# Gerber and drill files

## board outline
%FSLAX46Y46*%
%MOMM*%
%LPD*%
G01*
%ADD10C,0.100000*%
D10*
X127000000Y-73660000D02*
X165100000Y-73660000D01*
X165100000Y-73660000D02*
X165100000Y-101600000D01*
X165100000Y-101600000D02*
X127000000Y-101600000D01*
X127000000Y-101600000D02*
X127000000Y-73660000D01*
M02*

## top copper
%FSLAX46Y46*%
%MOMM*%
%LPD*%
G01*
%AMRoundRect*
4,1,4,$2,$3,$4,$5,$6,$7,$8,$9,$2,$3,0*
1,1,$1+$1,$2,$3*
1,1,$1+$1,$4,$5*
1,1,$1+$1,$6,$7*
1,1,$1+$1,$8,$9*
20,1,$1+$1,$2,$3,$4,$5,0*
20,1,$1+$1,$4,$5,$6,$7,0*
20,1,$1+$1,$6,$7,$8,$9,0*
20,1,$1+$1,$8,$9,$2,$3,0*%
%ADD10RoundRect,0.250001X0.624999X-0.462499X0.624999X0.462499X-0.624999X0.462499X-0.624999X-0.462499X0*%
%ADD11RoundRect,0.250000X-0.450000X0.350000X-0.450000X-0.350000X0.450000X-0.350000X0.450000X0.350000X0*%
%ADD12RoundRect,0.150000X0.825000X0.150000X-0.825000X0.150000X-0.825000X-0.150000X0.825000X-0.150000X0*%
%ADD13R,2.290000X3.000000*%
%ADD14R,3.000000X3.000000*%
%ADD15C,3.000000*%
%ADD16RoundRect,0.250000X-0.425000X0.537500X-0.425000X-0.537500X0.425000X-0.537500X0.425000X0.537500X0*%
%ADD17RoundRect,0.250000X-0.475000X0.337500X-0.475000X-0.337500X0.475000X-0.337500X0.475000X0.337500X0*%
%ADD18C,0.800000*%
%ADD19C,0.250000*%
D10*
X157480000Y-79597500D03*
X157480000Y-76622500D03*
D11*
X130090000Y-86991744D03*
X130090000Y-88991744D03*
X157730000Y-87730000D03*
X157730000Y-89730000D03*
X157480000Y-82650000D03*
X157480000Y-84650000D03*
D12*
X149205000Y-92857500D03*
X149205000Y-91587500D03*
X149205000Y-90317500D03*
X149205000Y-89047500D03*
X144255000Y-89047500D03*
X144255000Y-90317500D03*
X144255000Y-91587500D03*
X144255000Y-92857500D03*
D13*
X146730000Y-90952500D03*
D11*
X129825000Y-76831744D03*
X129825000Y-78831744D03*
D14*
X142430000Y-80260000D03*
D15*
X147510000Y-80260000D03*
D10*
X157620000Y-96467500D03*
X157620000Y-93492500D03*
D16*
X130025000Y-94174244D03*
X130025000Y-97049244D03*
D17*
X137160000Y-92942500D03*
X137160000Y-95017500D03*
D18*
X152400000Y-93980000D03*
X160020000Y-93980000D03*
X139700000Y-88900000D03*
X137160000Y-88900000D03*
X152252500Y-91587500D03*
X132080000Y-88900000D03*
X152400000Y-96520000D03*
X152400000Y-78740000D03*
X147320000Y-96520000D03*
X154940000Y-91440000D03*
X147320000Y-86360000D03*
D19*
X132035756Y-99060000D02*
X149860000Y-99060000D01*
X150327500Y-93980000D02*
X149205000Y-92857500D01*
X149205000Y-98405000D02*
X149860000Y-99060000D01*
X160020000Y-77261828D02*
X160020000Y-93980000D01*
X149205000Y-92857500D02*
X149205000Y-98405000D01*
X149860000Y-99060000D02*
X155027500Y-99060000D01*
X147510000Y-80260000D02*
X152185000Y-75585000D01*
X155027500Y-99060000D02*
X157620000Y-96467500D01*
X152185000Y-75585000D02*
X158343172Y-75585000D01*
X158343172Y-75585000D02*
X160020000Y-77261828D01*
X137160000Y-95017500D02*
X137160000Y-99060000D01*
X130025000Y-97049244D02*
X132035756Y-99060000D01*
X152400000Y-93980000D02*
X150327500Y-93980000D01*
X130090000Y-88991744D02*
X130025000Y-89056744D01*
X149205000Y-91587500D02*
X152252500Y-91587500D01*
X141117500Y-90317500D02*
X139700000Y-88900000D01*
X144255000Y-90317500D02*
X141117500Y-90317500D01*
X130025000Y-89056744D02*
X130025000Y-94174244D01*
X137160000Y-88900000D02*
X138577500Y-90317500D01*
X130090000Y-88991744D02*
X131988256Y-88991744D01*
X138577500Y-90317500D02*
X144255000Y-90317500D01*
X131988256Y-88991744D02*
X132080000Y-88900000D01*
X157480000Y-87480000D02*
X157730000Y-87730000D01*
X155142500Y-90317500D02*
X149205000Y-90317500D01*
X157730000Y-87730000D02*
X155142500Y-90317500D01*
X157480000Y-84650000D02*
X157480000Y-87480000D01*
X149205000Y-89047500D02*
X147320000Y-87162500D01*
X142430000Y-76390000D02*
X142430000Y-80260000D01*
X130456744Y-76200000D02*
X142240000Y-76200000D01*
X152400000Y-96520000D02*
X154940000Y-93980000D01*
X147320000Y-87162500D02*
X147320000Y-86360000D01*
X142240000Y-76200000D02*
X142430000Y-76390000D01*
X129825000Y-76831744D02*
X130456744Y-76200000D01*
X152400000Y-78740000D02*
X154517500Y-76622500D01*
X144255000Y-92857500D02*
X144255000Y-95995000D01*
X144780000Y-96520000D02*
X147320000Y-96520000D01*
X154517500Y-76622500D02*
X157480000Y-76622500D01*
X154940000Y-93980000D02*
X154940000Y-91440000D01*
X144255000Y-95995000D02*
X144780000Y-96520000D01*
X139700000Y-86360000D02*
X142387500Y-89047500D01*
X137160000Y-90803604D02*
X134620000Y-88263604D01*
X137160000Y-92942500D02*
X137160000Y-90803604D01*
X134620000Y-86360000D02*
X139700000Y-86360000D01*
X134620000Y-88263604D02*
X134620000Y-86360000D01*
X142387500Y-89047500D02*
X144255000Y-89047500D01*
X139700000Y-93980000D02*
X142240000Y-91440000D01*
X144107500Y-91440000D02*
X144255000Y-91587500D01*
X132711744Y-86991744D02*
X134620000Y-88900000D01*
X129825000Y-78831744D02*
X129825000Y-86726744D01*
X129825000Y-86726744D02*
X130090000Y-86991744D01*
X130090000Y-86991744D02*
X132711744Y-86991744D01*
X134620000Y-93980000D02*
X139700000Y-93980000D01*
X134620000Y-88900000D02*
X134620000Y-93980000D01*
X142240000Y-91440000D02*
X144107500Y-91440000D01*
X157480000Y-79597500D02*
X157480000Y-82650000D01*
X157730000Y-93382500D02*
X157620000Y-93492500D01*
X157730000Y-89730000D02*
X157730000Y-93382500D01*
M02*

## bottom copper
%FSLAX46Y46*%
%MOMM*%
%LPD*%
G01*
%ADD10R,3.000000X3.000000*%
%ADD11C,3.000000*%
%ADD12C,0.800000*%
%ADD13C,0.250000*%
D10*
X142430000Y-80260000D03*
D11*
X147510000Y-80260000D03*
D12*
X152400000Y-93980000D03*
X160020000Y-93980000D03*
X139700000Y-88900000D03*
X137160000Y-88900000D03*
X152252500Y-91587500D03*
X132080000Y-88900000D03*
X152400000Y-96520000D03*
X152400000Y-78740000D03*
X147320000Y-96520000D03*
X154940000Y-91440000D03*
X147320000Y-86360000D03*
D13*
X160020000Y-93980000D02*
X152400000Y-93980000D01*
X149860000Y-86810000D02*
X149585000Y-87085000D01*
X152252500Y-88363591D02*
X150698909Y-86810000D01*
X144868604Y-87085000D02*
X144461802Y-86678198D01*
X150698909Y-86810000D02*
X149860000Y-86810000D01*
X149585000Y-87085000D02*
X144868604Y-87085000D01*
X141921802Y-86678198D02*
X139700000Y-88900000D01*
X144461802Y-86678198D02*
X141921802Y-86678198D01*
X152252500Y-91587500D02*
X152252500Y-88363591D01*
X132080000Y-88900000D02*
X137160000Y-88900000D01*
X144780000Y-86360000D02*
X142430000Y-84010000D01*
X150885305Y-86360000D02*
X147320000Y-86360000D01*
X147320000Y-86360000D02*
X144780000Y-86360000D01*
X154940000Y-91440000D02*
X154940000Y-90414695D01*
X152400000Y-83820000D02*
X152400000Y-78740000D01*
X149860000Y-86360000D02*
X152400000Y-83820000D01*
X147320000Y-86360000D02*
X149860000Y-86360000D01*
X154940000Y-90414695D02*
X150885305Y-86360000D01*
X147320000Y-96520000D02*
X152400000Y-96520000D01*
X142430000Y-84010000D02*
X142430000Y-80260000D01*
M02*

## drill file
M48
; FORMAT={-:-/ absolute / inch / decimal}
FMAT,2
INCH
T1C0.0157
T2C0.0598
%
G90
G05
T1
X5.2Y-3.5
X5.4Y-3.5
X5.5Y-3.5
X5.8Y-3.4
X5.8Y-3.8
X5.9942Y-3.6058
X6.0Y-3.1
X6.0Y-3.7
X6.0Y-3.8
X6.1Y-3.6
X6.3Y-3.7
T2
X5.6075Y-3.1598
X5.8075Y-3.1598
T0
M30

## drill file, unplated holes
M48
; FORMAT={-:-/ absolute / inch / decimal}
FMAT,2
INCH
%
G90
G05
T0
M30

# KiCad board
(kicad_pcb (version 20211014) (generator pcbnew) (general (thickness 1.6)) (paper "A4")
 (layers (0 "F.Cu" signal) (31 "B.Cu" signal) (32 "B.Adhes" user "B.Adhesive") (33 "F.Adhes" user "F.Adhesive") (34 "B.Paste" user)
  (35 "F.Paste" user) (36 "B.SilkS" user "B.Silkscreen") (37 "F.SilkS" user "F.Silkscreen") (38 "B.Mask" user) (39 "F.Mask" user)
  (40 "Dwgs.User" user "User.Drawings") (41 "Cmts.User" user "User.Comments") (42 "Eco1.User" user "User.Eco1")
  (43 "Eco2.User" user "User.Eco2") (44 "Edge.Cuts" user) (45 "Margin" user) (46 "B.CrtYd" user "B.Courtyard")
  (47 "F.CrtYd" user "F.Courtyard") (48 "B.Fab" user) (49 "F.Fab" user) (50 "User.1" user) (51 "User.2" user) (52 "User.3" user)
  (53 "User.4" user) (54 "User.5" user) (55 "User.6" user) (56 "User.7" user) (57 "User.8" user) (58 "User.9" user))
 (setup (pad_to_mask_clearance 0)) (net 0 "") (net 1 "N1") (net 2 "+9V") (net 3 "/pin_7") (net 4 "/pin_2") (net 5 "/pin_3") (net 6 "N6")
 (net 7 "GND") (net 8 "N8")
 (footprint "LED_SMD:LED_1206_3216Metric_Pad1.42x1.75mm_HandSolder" (layer "F.Cu") (at 157.48 78.11 90)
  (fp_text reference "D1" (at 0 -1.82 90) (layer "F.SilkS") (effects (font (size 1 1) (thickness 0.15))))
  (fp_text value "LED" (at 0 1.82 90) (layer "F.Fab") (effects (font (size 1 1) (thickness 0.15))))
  (pad "1" smd roundrect (at -1.4875 0 90) (size 1.425 1.75) (layers "F.Cu" "F.Paste" "F.Mask") (roundrect_rratio 0.1754392982) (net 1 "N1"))
  (pad "2" smd roundrect (at 1.4875 0 90) (size 1.425 1.75) (layers "F.Cu" "F.Paste" "F.Mask") (roundrect_rratio 0.1754392982) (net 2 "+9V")))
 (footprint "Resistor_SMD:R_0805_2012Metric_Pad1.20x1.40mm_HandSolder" (layer "F.Cu") (at 130.09 87.991744 -90)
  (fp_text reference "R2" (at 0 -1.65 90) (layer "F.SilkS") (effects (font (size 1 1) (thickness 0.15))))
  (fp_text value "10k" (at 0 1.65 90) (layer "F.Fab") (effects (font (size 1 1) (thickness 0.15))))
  (pad "1" smd roundrect (at -1 0 270) (size 1.2 1.4) (layers "F.Cu" "F.Paste" "F.Mask") (roundrect_rratio 0.2083333333) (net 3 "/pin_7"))
  (pad "2" smd roundrect (at 1 0 270) (size 1.2 1.4) (layers "F.Cu" "F.Paste" "F.Mask") (roundrect_rratio 0.2083333333) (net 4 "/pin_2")))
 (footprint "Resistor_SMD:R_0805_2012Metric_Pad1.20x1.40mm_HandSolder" (layer "F.Cu") (at 157.73 88.73 -90)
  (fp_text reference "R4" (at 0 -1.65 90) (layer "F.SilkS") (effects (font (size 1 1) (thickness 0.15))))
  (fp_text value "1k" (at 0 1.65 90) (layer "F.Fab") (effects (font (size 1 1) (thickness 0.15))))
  (pad "1" smd roundrect (at -1 0 270) (size 1.2 1.4) (layers "F.Cu" "F.Paste" "F.Mask") (roundrect_rratio 0.2083333333) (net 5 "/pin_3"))
  (pad "2" smd roundrect (at 1 0 270) (size 1.2 1.4) (layers "F.Cu" "F.Paste" "F.Mask") (roundrect_rratio 0.2083333333) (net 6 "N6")))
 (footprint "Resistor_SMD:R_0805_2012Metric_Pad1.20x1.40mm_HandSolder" (layer "F.Cu") (at 157.48 83.65 -90)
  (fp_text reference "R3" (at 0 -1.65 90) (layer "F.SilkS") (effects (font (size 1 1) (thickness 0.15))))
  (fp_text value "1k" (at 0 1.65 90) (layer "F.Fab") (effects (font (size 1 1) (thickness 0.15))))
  (pad "1" smd roundrect (at -1 0 270) (size 1.2 1.4) (layers "F.Cu" "F.Paste" "F.Mask") (roundrect_rratio 0.2083333333) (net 1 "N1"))
  (pad "2" smd roundrect (at 1 0 270) (size 1.2 1.4) (layers "F.Cu" "F.Paste" "F.Mask") (roundrect_rratio 0.2083333333) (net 5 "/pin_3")))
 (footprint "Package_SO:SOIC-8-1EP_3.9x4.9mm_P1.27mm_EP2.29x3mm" (layer "F.Cu") (at 146.73 90.9525 180)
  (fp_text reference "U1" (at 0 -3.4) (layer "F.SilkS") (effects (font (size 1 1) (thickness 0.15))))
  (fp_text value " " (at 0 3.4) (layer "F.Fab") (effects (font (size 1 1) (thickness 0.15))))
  (pad "" smd roundrect (at -0.57 0.75 180) (size 0.92 1.21) (layers "F.Paste") (roundrect_rratio 0.25))
  (pad "" smd roundrect (at 0.57 -0.75 180) (size 0.92 1.21) (layers "F.Paste") (roundrect_rratio 0.25))
  (pad "" smd roundrect (at -0.57 -0.75 180) (size 0.92 1.21) (layers "F.Paste") (roundrect_rratio 0.25))
  (pad "" smd roundrect (at 0.57 0.75 180) (size 0.92 1.21) (layers "F.Paste") (roundrect_rratio 0.25))
  (pad "1" smd roundrect (at -2.475 -1.905 180) (size 1.95 0.6) (layers "F.Cu" "F.Paste" "F.Mask") (roundrect_rratio 0.25) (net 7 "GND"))
  (pad "2" smd roundrect (at -2.475 -0.635 180) (size 1.95 0.6) (layers "F.Cu" "F.Paste" "F.Mask") (roundrect_rratio 0.25) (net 4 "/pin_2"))
  (pad "3" smd roundrect (at -2.475 0.635 180) (size 1.95 0.6) (layers "F.Cu" "F.Paste" "F.Mask") (roundrect_rratio 0.25) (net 5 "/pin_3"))
  (pad "4" smd roundrect (at -2.475 1.905 180) (size 1.95 0.6) (layers "F.Cu" "F.Paste" "F.Mask") (roundrect_rratio 0.25) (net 2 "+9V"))
  (pad "5" smd roundrect (at 2.475 1.905 180) (size 1.95 0.6) (layers "F.Cu" "F.Paste" "F.Mask") (roundrect_rratio 0.25) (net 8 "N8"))
  (pad "6" smd roundrect (at 2.475 0.635 180) (size 1.95 0.6) (layers "F.Cu" "F.Paste" "F.Mask") (roundrect_rratio 0.25) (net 4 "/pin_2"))
  (pad "7" smd roundrect (at 2.475 -0.635 180) (size 1.95 0.6) (layers "F.Cu" "F.Paste" "F.Mask") (roundrect_rratio 0.25) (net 3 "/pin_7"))
  (pad "8" smd roundrect (at 2.475 -1.905 180) (size 1.95 0.6) (layers "F.Cu" "F.Paste" "F.Mask") (roundrect_rratio 0.25) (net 2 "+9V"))
  (pad "9" smd rect (at 0 0 180) (size 2.29 3) (layers "F.Cu" "F.Mask")))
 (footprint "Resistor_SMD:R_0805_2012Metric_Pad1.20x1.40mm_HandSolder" (layer "F.Cu") (at 129.825 77.831744 -90)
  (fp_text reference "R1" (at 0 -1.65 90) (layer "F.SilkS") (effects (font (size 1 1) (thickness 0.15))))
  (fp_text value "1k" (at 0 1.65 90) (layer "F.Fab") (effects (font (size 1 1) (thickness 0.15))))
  (pad "1" smd roundrect (at -1 0 270) (size 1.2 1.4) (layers "F.Cu" "F.Paste" "F.Mask") (roundrect_rratio 0.2083333333) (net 2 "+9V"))
  (pad "2" smd roundrect (at 1 0 270) (size 1.2 1.4) (layers "F.Cu" "F.Paste" "F.Mask") (roundrect_rratio 0.2083333333) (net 3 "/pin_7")))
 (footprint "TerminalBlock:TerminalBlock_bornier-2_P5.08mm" (layer "F.Cu") (at 142.43 80.26)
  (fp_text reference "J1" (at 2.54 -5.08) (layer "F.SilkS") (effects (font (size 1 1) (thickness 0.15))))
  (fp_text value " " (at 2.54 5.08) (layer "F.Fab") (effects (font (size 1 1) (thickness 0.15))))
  (pad "1" thru_hole rect (at 0 0) (size 3 3) (drill 1.52) (layers *.Cu *.Mask) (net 2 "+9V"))
  (pad "2" thru_hole circle (at 5.08 0) (size 3 3) (drill 1.52) (layers *.Cu *.Mask) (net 7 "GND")))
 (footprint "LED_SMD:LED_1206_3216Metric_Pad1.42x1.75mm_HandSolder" (layer "F.Cu") (at 157.62 94.98 90)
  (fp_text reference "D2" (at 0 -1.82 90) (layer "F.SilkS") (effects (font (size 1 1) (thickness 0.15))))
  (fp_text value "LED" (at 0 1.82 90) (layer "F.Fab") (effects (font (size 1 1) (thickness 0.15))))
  (pad "1" smd roundrect (at -1.4875 0 90) (size 1.425 1.75) (layers "F.Cu" "F.Paste" "F.Mask") (roundrect_rratio 0.1754392982)
   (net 7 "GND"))
  (pad "2" smd roundrect (at 1.4875 0 90) (size 1.425 1.75) (layers "F.Cu" "F.Paste" "F.Mask") (roundrect_rratio 0.1754392982) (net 6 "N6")))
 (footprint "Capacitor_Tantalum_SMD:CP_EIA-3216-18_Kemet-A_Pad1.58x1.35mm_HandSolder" (layer "F.Cu") (at 130.025 95.611744 -90)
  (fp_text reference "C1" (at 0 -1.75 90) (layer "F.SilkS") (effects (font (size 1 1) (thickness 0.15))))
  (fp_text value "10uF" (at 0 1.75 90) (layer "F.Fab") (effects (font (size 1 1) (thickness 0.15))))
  (pad "1" smd roundrect (at -1.4375 0 270) (size 1.575 1.35) (layers "F.Cu" "F.Paste" "F.Mask") (roundrect_rratio 0.1851851852)
   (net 4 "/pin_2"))
  (pad "2" smd roundrect (at 1.4375 0 270) (size 1.575 1.35) (layers "F.Cu" "F.Paste" "F.Mask") (roundrect_rratio 0.1851851852)
   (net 7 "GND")))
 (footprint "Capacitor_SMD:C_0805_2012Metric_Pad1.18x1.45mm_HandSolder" (layer "F.Cu") (at 137.16 93.98 -90)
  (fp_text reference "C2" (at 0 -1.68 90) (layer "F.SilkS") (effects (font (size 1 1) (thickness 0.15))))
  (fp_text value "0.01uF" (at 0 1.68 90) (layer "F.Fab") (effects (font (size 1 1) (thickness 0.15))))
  (pad "1" smd roundrect (at -1.0375 0 270) (size 1.175 1.45) (layers "F.Cu" "F.Paste" "F.Mask") (roundrect_rratio 0.2127659574)
   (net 8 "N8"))
  (pad "2" smd roundrect (at 1.0375 0 270) (size 1.175 1.45) (layers "F.Cu" "F.Paste" "F.Mask") (roundrect_rratio 0.2127659574)
   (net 7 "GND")))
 (gr_rect (start 127 73.66) (end 165.1 101.6) (layer "Edge.Cuts") (width 0.1) (fill none))
 (segment (start 132.035756 99.06) (end 149.86 99.06) (width 0.25) (layer "F.Cu") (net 7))
 (segment (start 150.3275 93.98) (end 149.205 92.8575) (width 0.25) (layer "F.Cu") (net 7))
 (segment (start 149.205 98.405) (end 149.86 99.06) (width 0.25) (layer "F.Cu") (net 7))
 (segment (start 160.02 77.261828) (end 160.02 93.98) (width 0.25) (layer "F.Cu") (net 7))
 (segment (start 149.205 92.8575) (end 149.205 98.405) (width 0.25) (layer "F.Cu") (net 7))
 (segment (start 149.86 99.06) (end 155.0275 99.06) (width 0.25) (layer "F.Cu") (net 7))
 (segment (start 147.51 80.26) (end 152.185 75.585) (width 0.25) (layer "F.Cu") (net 7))
 (segment (start 155.0275 99.06) (end 157.62 96.4675) (width 0.25) (layer "F.Cu") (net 7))
 (segment (start 152.185 75.585) (end 158.343172 75.585) (width 0.25) (layer "F.Cu") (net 7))
 (segment (start 158.343172 75.585) (end 160.02 77.261828) (width 0.25) (layer "F.Cu") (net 7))
 (segment (start 137.16 95.0175) (end 137.16 99.06) (width 0.25) (layer "F.Cu") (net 7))
 (segment (start 130.025 97.049244) (end 132.035756 99.06) (width 0.25) (layer "F.Cu") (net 7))
 (segment (start 152.4 93.98) (end 150.3275 93.98) (width 0.25) (layer "F.Cu") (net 7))
 (via (at 152.4 93.98) (size 0.8) (drill 0.4) (layers "F.Cu" "B.Cu") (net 7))
 (via (at 160.02 93.98) (size 0.8) (drill 0.4) (layers "F.Cu" "B.Cu") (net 7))
 (segment (start 160.02 93.98) (end 152.4 93.98) (width 0.25) (layer "B.Cu") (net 7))
 (segment (start 130.09 88.991744) (end 130.025 89.056744) (width 0.25) (layer "F.Cu") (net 4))
 (segment (start 149.205 91.5875) (end 152.2525 91.5875) (width 0.25) (layer "F.Cu") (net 4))
 (segment (start 141.1175 90.3175) (end 139.7 88.9) (width 0.25) (layer "F.Cu") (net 4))
 (segment (start 144.255 90.3175) (end 141.1175 90.3175) (width 0.25) (layer "F.Cu") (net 4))
 (segment (start 130.025 89.056744) (end 130.025 94.174244) (width 0.25) (layer "F.Cu") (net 4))
 (segment (start 137.16 88.9) (end 138.5775 90.3175) (width 0.25) (layer "F.Cu") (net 4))
 (segment (start 130.09 88.991744) (end 131.988256 88.991744) (width 0.25) (layer "F.Cu") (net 4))
 (segment (start 138.5775 90.3175) (end 144.255 90.3175) (width 0.25) (layer "F.Cu") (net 4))
 (segment (start 131.988256 88.991744) (end 132.08 88.9) (width 0.25) (layer "F.Cu") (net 4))
 (via (at 139.7 88.9) (size 0.8) (drill 0.4) (layers "F.Cu" "B.Cu") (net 4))
 (via (at 137.16 88.9) (size 0.8) (drill 0.4) (layers "F.Cu" "B.Cu") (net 4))
 (via (at 152.2525 91.5875) (size 0.8) (drill 0.4) (layers "F.Cu" "B.Cu") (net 4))
 (via (at 132.08 88.9) (size 0.8) (drill 0.4) (layers "F.Cu" "B.Cu") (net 4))
 (segment (start 149.86 86.81) (end 149.585 87.085) (width 0.25) (layer "B.Cu") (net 4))
 (segment (start 152.2525 88.363591) (end 150.698909 86.81) (width 0.25) (layer "B.Cu") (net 4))
 (segment (start 144.868604 87.085) (end 144.461802 86.678198) (width 0.25) (layer "B.Cu") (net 4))
 (segment (start 150.698909 86.81) (end 149.86 86.81) (width 0.25) (layer "B.Cu") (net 4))
 (segment (start 149.585 87.085) (end 144.868604 87.085) (width 0.25) (layer "B.Cu") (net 4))
 (segment (start 141.921802 86.678198) (end 139.7 88.9) (width 0.25) (layer "B.Cu") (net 4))
 (segment (start 144.461802 86.678198) (end 141.921802 86.678198) (width 0.25) (layer "B.Cu") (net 4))
 (segment (start 152.2525 91.5875) (end 152.2525 88.363591) (width 0.25) (layer "B.Cu") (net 4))
 (segment (start 132.08 88.9) (end 137.16 88.9) (width 0.25) (layer "B.Cu") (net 4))
 (segment (start 157.48 87.48) (end 157.73 87.73) (width 0.25) (layer "F.Cu") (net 5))
 (segment (start 155.1425 90.3175) (end 149.205 90.3175) (width 0.25) (layer "F.Cu") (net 5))
 (segment (start 157.73 87.73) (end 155.1425 90.3175) (width 0.25) (layer "F.Cu") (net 5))
 (segment (start 157.48 84.65) (end 157.48 87.48) (width 0.25) (layer "F.Cu") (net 5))
 (segment (start 149.205 89.0475) (end 147.32 87.1625) (width 0.25) (layer "F.Cu") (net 2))
 (segment (start 142.43 76.39) (end 142.43 80.26) (width 0.25) (layer "F.Cu") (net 2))
 (segment (start 130.456744 76.2) (end 142.24 76.2) (width 0.25) (layer "F.Cu") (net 2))
 (segment (start 152.4 96.52) (end 154.94 93.98) (width 0.25) (layer "F.Cu") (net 2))
 (segment (start 147.32 87.1625) (end 147.32 86.36) (width 0.25) (layer "F.Cu") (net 2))
 (segment (start 142.24 76.2) (end 142.43 76.39) (width 0.25) (layer "F.Cu") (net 2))
 (segment (start 129.825 76.831744) (end 130.456744 76.2) (width 0.25) (layer "F.Cu") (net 2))
 (segment (start 152.4 78.74) (end 154.5175 76.6225) (width 0.25) (layer "F.Cu") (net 2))
 (segment (start 144.255 92.8575) (end 144.255 95.995) (width 0.25) (layer "F.Cu") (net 2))
 (segment (start 144.78 96.52) (end 147.32 96.52) (width 0.25) (layer "F.Cu") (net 2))
 (segment (start 154.5175 76.6225) (end 157.48 76.6225) (width 0.25) (layer "F.Cu") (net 2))
 (segment (start 154.94 93.98) (end 154.94 91.44) (width 0.25) (layer "F.Cu") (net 2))
 (segment (start 144.255 95.995) (end 144.78 96.52) (width 0.25) (layer "F.Cu") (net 2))
 (via (at 152.4 96.52) (size 0.8) (drill 0.4) (layers "F.Cu" "B.Cu") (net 2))
 (via (at 152.4 78.74) (size 0.8) (drill 0.4) (layers "F.Cu" "B.Cu") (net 2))
 (via (at 147.32 96.52) (size 0.8) (drill 0.4) (layers "F.Cu" "B.Cu") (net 2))
 (via (at 154.94 91.44) (size 0.8) (drill 0.4) (layers "F.Cu" "B.Cu") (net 2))
 (via (at 147.32 86.36) (size 0.8) (drill 0.4) (layers "F.Cu" "B.Cu") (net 2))
 (segment (start 144.78 86.36) (end 142.43 84.01) (width 0.25) (layer "B.Cu") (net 2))
 (segment (start 150.885305 86.36) (end 147.32 86.36) (width 0.25) (layer "B.Cu") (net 2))
 (segment (start 147.32 86.36) (end 144.78 86.36) (width 0.25) (layer "B.Cu") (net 2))
 (segment (start 154.94 91.44) (end 154.94 90.414695) (width 0.25) (layer "B.Cu") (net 2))
 (segment (start 152.4 83.82) (end 152.4 78.74) (width 0.25) (layer "B.Cu") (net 2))
 (segment (start 149.86 86.36) (end 152.4 83.82) (width 0.25) (layer "B.Cu") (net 2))
 (segment (start 147.32 86.36) (end 149.86 86.36) (width 0.25) (layer "B.Cu") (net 2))
 (segment (start 154.94 90.414695) (end 150.885305 86.36) (width 0.25) (layer "B.Cu") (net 2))
 (segment (start 147.32 96.52) (end 152.4 96.52) (width 0.25) (layer "B.Cu") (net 2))
 (segment (start 142.43 84.01) (end 142.43 80.26) (width 0.25) (layer "B.Cu") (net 2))
 (segment (start 139.7 86.36) (end 142.3875 89.0475) (width 0.25) (layer "F.Cu") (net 8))
 (segment (start 137.16 90.803604) (end 134.62 88.263604) (width 0.25) (layer "F.Cu") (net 8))
 (segment (start 137.16 92.9425) (end 137.16 90.803604) (width 0.25) (layer "F.Cu") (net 8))
 (segment (start 134.62 86.36) (end 139.7 86.36) (width 0.25) (layer "F.Cu") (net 8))
 (segment (start 134.62 88.263604) (end 134.62 86.36) (width 0.25) (layer "F.Cu") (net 8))
 (segment (start 142.3875 89.0475) (end 144.255 89.0475) (width 0.25) (layer "F.Cu") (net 8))
 (segment (start 139.7 93.98) (end 142.24 91.44) (width 0.25) (layer "F.Cu") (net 3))
 (segment (start 144.1075 91.44) (end 144.255 91.5875) (width 0.25) (layer "F.Cu") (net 3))
 (segment (start 132.711744 86.991744) (end 134.62 88.9) (width 0.25) (layer "F.Cu") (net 3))
 (segment (start 129.825 78.831744) (end 129.825 86.726744) (width 0.25) (layer "F.Cu") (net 3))
 (segment (start 129.825 86.726744) (end 130.09 86.991744) (width 0.25) (layer "F.Cu") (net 3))
 (segment (start 130.09 86.991744) (end 132.711744 86.991744) (width 0.25) (layer "F.Cu") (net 3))
 (segment (start 134.62 93.98) (end 139.7 93.98) (width 0.25) (layer "F.Cu") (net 3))
 (segment (start 134.62 88.9) (end 134.62 93.98) (width 0.25) (layer "F.Cu") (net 3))
 (segment (start 142.24 91.44) (end 144.1075 91.44) (width 0.25) (layer "F.Cu") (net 3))
 (segment (start 157.48 79.5975) (end 157.48 82.65) (width 0.25) (layer "F.Cu") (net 1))
 (segment (start 157.73 93.3825) (end 157.62 93.4925) (width 0.25) (layer "F.Cu") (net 6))
 (segment (start 157.73 89.73) (end 157.73 93.3825) (width 0.25) (layer "F.Cu") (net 6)))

